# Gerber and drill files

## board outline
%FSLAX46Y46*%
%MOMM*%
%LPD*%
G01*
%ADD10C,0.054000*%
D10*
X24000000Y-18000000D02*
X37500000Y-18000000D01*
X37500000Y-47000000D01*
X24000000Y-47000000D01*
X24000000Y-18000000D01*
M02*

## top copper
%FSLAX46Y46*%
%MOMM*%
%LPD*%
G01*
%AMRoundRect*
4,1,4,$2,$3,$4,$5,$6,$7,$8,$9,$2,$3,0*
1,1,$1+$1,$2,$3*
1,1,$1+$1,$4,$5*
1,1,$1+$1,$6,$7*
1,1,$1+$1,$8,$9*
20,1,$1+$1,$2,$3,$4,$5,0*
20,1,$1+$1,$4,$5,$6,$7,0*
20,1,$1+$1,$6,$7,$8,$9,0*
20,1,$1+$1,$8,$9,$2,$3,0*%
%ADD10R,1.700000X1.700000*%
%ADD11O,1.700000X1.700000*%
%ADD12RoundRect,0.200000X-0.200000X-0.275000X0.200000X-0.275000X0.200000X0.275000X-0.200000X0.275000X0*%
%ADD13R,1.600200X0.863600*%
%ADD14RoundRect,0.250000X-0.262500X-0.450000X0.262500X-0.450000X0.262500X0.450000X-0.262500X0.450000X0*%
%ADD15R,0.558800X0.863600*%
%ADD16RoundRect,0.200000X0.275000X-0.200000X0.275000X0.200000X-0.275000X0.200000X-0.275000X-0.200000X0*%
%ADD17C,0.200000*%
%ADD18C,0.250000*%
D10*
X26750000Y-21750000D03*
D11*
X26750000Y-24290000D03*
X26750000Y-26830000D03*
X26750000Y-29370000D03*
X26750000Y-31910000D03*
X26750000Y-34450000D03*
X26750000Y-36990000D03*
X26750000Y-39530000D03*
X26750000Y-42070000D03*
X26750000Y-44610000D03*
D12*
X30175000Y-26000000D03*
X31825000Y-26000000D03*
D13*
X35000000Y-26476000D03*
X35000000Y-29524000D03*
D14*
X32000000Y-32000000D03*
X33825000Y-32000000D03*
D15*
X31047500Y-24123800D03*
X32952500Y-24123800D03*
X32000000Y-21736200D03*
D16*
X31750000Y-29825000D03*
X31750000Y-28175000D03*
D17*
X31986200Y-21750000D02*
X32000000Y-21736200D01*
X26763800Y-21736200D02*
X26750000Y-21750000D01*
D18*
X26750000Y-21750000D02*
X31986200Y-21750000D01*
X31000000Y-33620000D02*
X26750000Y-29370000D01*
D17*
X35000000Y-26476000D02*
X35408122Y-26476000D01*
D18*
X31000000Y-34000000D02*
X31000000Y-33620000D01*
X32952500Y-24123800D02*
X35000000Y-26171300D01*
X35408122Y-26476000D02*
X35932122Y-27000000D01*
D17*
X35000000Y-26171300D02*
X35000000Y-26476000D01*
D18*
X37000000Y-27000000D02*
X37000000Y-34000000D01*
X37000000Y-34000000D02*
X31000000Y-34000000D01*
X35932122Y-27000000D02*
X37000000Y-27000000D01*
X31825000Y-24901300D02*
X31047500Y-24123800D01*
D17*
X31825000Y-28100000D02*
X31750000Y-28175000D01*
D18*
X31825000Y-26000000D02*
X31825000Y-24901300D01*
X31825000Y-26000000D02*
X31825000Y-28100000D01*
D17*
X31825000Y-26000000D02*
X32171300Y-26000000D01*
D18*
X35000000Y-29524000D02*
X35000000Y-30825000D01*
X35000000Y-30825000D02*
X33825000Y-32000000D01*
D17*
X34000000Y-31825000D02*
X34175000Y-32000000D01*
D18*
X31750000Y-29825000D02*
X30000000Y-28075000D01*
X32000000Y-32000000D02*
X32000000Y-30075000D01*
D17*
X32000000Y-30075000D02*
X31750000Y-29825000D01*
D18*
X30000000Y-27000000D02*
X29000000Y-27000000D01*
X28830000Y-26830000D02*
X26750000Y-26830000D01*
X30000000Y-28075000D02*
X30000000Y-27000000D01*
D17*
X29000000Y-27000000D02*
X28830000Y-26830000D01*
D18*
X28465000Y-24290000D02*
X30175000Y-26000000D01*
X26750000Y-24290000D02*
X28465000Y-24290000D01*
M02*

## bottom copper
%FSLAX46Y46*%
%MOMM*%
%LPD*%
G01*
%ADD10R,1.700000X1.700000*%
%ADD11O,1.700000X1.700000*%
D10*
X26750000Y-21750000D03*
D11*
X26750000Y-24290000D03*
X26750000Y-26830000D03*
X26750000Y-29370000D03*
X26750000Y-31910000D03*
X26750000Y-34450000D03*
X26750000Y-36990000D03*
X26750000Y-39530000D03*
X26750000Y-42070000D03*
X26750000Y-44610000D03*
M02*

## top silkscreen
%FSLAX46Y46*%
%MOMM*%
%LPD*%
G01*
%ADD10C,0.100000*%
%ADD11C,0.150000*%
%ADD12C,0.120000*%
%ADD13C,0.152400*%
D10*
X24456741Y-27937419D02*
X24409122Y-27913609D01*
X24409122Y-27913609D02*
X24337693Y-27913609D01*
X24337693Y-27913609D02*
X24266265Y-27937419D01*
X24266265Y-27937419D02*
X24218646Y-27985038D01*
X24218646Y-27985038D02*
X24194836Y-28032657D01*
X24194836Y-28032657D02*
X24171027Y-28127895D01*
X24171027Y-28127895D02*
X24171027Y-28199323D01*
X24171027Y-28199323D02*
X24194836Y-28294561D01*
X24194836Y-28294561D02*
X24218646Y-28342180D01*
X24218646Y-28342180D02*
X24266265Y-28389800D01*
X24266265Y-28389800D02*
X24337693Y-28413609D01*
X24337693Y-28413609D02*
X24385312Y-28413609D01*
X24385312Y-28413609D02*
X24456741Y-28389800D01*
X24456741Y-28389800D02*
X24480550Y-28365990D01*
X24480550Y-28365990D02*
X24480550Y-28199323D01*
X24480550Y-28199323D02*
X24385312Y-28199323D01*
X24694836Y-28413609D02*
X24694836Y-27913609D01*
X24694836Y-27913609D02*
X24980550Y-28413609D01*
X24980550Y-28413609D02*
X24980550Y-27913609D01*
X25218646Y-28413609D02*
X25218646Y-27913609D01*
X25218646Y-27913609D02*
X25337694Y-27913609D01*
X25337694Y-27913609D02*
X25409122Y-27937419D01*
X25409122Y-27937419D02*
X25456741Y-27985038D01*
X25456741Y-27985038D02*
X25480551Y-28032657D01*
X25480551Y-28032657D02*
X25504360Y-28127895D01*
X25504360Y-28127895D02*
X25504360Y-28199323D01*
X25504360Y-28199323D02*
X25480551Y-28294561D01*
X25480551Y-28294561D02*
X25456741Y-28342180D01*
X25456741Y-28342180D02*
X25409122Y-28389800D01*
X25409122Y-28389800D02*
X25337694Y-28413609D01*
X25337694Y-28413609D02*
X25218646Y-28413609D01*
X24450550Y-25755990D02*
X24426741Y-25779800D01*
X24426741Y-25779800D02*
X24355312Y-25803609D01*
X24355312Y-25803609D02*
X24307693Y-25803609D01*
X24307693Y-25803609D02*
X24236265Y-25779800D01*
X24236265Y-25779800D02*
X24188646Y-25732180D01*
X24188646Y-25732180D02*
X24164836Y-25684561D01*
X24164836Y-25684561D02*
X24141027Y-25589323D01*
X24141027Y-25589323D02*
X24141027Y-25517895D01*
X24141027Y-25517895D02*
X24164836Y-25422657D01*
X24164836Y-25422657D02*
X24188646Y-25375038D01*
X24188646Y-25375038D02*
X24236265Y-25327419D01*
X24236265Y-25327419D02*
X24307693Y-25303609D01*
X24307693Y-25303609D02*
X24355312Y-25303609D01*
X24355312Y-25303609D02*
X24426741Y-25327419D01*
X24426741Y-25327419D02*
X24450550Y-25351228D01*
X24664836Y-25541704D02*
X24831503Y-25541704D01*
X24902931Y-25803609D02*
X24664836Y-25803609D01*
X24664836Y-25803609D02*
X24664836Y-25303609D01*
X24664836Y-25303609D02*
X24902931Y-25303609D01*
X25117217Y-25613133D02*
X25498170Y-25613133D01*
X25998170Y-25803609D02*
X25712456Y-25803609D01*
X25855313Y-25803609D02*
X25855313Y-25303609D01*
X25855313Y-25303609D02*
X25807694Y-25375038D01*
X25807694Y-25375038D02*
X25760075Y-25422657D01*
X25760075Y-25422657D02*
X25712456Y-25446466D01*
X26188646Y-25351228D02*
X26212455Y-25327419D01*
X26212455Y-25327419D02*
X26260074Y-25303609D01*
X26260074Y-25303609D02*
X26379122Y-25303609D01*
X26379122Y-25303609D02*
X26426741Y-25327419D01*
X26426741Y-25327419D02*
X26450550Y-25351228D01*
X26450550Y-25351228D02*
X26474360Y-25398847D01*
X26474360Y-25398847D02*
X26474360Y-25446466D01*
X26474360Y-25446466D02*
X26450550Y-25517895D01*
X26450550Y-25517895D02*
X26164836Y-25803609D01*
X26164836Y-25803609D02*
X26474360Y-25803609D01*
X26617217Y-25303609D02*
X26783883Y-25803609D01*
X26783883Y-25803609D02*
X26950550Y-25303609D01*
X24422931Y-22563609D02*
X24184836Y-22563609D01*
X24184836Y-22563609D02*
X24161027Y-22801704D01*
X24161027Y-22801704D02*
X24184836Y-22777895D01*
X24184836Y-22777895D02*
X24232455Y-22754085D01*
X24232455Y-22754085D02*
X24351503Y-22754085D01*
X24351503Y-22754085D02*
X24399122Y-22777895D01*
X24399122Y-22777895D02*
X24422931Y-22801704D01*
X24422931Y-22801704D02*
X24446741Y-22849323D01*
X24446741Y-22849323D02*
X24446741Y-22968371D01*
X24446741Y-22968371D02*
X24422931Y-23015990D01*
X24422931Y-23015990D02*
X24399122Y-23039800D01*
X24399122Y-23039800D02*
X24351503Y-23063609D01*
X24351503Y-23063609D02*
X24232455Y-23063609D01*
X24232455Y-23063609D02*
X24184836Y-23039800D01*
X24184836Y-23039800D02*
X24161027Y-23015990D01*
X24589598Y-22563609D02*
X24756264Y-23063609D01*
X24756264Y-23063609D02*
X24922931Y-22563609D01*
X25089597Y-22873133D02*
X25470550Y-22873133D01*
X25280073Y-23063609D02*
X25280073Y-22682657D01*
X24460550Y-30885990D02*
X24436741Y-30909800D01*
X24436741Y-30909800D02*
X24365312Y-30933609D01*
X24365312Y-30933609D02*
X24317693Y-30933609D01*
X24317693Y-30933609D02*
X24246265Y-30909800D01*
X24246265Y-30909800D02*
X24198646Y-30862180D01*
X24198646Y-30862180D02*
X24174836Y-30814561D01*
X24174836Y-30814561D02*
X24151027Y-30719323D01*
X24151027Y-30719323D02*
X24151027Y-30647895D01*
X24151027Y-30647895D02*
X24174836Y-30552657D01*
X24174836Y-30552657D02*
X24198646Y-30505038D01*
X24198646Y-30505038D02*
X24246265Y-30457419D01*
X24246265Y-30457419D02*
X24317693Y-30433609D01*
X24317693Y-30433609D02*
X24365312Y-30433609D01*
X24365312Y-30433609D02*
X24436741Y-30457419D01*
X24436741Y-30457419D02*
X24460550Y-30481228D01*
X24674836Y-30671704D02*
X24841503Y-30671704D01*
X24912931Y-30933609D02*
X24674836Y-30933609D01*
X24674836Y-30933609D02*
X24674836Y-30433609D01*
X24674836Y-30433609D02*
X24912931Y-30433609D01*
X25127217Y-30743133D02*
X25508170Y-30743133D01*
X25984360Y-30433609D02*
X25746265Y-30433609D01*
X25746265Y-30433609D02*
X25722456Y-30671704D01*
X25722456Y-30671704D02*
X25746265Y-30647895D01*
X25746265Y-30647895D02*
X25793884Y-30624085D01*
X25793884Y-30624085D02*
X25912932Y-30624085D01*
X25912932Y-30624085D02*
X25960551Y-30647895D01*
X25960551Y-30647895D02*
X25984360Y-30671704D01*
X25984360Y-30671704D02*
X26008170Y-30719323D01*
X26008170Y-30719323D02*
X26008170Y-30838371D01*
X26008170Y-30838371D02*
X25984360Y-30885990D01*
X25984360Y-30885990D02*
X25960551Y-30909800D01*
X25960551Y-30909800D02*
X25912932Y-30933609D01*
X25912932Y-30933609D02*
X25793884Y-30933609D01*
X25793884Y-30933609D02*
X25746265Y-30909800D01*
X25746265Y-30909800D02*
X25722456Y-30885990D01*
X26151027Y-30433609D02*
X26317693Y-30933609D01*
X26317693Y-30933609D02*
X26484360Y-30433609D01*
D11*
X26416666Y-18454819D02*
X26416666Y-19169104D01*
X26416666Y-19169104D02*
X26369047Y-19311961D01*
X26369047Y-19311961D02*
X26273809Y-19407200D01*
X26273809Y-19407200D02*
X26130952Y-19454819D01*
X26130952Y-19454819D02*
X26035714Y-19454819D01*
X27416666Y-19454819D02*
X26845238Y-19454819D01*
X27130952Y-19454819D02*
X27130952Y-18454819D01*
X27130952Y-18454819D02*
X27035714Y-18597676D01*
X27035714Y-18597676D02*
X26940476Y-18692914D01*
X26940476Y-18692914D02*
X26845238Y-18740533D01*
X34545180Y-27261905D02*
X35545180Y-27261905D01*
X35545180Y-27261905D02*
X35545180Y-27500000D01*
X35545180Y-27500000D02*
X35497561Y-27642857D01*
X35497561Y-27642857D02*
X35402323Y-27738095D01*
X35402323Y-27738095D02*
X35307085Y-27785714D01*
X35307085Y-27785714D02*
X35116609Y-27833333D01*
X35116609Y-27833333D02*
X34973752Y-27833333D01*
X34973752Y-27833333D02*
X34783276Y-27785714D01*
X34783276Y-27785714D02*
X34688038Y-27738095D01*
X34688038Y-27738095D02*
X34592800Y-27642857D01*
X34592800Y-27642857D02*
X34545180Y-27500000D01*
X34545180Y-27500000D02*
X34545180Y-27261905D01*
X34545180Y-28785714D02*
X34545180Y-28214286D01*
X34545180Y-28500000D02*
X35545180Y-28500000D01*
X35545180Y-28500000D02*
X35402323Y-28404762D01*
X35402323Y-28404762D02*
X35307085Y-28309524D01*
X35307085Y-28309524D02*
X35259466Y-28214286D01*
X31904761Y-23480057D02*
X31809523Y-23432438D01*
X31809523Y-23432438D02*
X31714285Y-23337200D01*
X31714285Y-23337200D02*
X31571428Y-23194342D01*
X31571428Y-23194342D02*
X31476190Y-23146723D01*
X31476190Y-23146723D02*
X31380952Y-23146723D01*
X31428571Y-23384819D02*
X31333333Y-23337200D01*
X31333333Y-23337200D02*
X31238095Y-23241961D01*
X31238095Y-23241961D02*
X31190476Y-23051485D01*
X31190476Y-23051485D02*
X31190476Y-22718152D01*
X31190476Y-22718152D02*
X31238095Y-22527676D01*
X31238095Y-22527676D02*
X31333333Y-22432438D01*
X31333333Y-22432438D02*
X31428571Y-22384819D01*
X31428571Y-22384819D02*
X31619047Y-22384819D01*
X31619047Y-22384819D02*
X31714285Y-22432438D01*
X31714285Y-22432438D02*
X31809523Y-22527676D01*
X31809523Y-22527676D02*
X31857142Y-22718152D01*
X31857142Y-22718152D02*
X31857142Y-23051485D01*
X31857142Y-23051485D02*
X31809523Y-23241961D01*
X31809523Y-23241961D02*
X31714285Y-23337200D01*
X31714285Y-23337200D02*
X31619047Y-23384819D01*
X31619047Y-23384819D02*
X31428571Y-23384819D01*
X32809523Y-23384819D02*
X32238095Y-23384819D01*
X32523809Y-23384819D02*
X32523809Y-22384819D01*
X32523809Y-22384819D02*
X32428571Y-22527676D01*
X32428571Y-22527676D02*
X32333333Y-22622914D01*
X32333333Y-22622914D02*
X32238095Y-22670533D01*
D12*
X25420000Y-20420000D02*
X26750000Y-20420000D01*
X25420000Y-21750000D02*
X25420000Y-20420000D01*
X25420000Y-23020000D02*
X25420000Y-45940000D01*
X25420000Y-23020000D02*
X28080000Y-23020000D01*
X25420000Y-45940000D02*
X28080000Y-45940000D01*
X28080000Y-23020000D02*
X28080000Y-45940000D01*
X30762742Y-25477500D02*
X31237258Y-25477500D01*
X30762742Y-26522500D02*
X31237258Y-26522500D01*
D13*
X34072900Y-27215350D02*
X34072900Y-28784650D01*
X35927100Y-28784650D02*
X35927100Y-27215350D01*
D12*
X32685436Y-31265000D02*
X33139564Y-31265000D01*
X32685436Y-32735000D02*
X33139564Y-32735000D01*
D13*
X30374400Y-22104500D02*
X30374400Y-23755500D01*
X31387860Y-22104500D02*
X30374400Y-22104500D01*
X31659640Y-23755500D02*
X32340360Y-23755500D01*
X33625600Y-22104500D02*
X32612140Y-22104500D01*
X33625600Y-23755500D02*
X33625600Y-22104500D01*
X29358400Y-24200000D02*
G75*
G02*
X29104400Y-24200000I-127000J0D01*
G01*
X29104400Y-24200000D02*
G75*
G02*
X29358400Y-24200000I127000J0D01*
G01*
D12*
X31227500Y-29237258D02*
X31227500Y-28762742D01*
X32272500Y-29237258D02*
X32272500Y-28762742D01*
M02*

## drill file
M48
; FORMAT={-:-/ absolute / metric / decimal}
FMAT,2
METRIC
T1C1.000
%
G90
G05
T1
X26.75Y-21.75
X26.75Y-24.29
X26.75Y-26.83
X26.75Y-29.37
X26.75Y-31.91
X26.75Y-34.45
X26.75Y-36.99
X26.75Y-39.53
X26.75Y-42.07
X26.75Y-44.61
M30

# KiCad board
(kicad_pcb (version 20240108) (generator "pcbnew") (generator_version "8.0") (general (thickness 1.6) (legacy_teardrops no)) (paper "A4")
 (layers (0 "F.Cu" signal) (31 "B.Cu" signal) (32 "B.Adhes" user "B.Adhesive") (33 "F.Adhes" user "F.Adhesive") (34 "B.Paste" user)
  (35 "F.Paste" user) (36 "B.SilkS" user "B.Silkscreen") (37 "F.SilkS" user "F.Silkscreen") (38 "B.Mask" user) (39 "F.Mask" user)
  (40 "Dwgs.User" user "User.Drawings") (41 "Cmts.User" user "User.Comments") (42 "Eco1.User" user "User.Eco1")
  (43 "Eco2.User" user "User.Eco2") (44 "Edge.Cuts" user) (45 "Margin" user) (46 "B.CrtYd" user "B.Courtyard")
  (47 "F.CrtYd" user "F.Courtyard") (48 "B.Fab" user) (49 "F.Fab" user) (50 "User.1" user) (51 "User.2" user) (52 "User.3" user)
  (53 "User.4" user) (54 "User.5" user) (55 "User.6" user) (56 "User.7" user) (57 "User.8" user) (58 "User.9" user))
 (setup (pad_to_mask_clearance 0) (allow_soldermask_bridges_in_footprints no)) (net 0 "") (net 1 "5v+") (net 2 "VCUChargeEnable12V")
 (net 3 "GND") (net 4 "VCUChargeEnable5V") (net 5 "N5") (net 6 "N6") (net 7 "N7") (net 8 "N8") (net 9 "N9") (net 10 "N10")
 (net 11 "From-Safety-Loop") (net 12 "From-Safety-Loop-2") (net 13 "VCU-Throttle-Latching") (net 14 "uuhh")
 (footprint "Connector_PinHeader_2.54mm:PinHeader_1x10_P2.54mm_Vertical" (layer "F.Cu") (at 26.75 21.75)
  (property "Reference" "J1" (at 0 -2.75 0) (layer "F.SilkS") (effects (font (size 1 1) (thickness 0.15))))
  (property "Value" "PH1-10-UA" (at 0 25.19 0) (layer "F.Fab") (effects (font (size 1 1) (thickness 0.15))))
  (fp_line (start -1.33 -1.33) (end 0 -1.33) (stroke (width 0.12) (type solid)) (layer "F.SilkS"))
  (fp_line (start -1.33 0) (end -1.33 -1.33) (stroke (width 0.12) (type solid)) (layer "F.SilkS"))
  (fp_line (start -1.33 1.27) (end -1.33 24.19) (stroke (width 0.12) (type solid)) (layer "F.SilkS"))
  (fp_line (start -1.33 1.27) (end 1.33 1.27) (stroke (width 0.12) (type solid)) (layer "F.SilkS"))
  (fp_line (start -1.33 24.19) (end 1.33 24.19) (stroke (width 0.12) (type solid)) (layer "F.SilkS"))
  (fp_line (start 1.33 1.27) (end 1.33 24.19) (stroke (width 0.12) (type solid)) (layer "F.SilkS"))
  (pad "1" thru_hole rect (at 0 0) (size 1.7 1.7) (drill 1) (layers "*.Cu" "*.Mask") (remove_unused_layers no) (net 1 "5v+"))
  (pad "2" thru_hole oval (at 0 2.54) (size 1.7 1.7) (drill 1) (layers "*.Cu" "*.Mask") (remove_unused_layers no)
   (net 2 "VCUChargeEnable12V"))
  (pad "3" thru_hole oval (at 0 5.08) (size 1.7 1.7) (drill 1) (layers "*.Cu" "*.Mask") (remove_unused_layers no) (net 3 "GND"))
  (pad "4" thru_hole oval (at 0 7.62) (size 1.7 1.7) (drill 1) (layers "*.Cu" "*.Mask") (remove_unused_layers no)
   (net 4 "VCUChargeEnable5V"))
  (pad "5" thru_hole oval (at 0 10.16) (size 1.7 1.7) (drill 1) (layers "*.Cu" "*.Mask") (remove_unused_layers no) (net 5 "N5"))
  (pad "6" thru_hole oval (at 0 12.7) (size 1.7 1.7) (drill 1) (layers "*.Cu" "*.Mask") (remove_unused_layers no) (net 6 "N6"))
  (pad "7" thru_hole oval (at 0 15.24) (size 1.7 1.7) (drill 1) (layers "*.Cu" "*.Mask") (remove_unused_layers no) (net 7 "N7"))
  (pad "8" thru_hole oval (at 0 17.78) (size 1.7 1.7) (drill 1) (layers "*.Cu" "*.Mask") (remove_unused_layers no) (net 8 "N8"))
  (pad "9" thru_hole oval (at 0 20.32) (size 1.7 1.7) (drill 1) (layers "*.Cu" "*.Mask") (remove_unused_layers no) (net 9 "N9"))
  (pad "10" thru_hole oval (at 0 22.86) (size 1.7 1.7) (drill 1) (layers "*.Cu" "*.Mask") (remove_unused_layers no) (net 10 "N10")))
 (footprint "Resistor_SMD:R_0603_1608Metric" (layer "F.Cu") (at 31 26)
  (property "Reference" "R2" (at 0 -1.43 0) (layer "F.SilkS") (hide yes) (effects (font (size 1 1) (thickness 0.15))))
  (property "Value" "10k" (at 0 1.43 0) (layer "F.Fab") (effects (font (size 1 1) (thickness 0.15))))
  (fp_line (start -0.237258 -0.5225) (end 0.237258 -0.5225) (stroke (width 0.12) (type solid)) (layer "F.SilkS"))
  (fp_line (start -0.237258 0.5225) (end 0.237258 0.5225) (stroke (width 0.12) (type solid)) (layer "F.SilkS"))
  (pad "1" smd roundrect (at -0.825 0) (size 0.8 0.95) (layers "F.Cu" "F.Paste" "F.Mask") (roundrect_rratio 0.25)
   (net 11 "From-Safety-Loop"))
  (pad "2" smd roundrect (at 0.825 0) (size 0.8 0.95) (layers "F.Cu" "F.Paste" "F.Mask") (roundrect_rratio 0.25)
   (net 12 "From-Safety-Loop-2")))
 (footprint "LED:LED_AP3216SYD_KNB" (layer "F.Cu") (at 35 28 -90)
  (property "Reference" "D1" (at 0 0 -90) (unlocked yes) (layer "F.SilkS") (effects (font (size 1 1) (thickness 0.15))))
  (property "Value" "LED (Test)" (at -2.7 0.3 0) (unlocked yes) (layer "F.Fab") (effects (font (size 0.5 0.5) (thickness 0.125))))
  (fp_line (start -0.78465 0.9271) (end 0.78465 0.9271) (stroke (width 0.1524) (type solid)) (layer "F.SilkS"))
  (fp_line (start 0.78465 -0.9271) (end -0.78465 -0.9271) (stroke (width 0.1524) (type solid)) (layer "F.SilkS"))
  (pad "1" smd rect (at -1.524 0 270) (size 0.8636 1.6002) (layers "F.Cu" "F.Paste" "F.Mask") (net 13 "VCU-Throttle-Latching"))
  (pad "2" smd rect (at 1.524 0 270) (size 0.8636 1.6002) (layers "F.Cu" "F.Paste" "F.Mask") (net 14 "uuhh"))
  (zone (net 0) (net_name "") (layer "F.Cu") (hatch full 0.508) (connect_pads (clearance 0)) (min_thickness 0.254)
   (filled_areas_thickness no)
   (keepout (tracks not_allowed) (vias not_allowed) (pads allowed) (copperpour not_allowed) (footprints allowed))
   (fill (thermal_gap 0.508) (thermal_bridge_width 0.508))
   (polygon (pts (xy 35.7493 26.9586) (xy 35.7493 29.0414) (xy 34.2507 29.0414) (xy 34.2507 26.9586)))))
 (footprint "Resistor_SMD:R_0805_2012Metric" (layer "F.Cu") (at 32.9125 32)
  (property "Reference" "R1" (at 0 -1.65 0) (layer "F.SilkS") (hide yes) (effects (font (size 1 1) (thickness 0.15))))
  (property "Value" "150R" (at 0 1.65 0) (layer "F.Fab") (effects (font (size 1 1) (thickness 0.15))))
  (fp_line (start -0.227064 -0.735) (end 0.227064 -0.735) (stroke (width 0.12) (type solid)) (layer "F.SilkS"))
  (fp_line (start -0.227064 0.735) (end 0.227064 0.735) (stroke (width 0.12) (type solid)) (layer "F.SilkS"))
  (pad "1" smd roundrect (at -0.9125 0) (size 1.025 1.4) (layers "F.Cu" "F.Paste" "F.Mask") (roundrect_rratio 0.243902) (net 3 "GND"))
  (pad "2" smd roundrect (at 0.9125 0) (size 1.025 1.4) (layers "F.Cu" "F.Paste" "F.Mask") (roundrect_rratio 0.243902) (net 14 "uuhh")))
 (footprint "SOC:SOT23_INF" (layer "F.Cu") (at 32 22.93)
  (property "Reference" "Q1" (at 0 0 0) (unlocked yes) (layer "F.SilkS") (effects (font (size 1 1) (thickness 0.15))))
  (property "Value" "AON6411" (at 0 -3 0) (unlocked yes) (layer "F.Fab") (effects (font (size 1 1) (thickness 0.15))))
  (fp_line (start -1.6256 -0.8255) (end -1.6256 0.8255) (stroke (width 0.1524) (type solid)) (layer "F.SilkS"))
  (fp_line (start -0.61214 -0.8255) (end -1.6256 -0.8255) (stroke (width 0.1524) (type solid)) (layer "F.SilkS"))
  (fp_line (start -0.34036 0.8255) (end 0.34036 0.8255) (stroke (width 0.1524) (type solid)) (layer "F.SilkS"))
  (fp_line (start 1.6256 -0.8255) (end 0.61214 -0.8255) (stroke (width 0.1524) (type solid)) (layer "F.SilkS"))
  (fp_line (start 1.6256 0.8255) (end 1.6256 -0.8255) (stroke (width 0.1524) (type solid)) (layer "F.SilkS"))
  (fp_circle (center -2.7686 1.27) (end -2.6416 1.27) (stroke (width 0.1524) (type solid)) (fill none) (layer "F.SilkS"))
  (pad "1" smd rect (at -0.9525 1.1938) (size 0.5588 0.8636) (layers "F.Cu" "F.Paste" "F.Mask") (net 12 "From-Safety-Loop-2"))
  (pad "2" smd rect (at 0.9525 1.1938) (size 0.5588 0.8636) (layers "F.Cu" "F.Paste" "F.Mask") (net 13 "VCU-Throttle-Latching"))
  (pad "3" smd rect (at 0 -1.1938) (size 0.5588 0.8636) (layers "F.Cu" "F.Paste" "F.Mask") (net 1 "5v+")))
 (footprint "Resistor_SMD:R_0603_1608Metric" (layer "F.Cu") (at 31.75 29 90)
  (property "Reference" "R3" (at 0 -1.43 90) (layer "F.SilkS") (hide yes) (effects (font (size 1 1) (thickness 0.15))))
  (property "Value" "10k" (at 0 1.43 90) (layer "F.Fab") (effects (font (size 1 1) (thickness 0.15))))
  (fp_line (start -0.237258 -0.5225) (end 0.237258 -0.5225) (stroke (width 0.12) (type solid)) (layer "F.SilkS"))
  (fp_line (start -0.237258 0.5225) (end 0.237258 0.5225) (stroke (width 0.12) (type solid)) (layer "F.SilkS"))
  (pad "1" smd roundrect (at -0.825 0 90) (size 0.8 0.95) (layers "F.Cu" "F.Paste" "F.Mask") (roundrect_rratio 0.25) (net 3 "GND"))
  (pad "2" smd roundrect (at 0.825 0 90) (size 0.8 0.95) (layers "F.Cu" "F.Paste" "F.Mask") (roundrect_rratio 0.25)
   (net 12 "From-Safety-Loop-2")))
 (gr_rect (start 24 18) (end 37.5 47) (stroke (width 0.054) (type default)) (fill none) (layer "Edge.Cuts"))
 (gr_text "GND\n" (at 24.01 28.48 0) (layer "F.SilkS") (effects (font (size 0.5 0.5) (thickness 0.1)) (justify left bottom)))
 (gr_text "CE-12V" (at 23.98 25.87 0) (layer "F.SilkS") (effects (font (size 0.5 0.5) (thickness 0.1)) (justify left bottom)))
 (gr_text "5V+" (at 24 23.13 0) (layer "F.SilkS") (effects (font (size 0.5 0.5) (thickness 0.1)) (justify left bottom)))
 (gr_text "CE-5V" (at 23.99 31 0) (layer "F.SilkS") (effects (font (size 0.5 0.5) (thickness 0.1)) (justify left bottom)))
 (segment (start 31.9862 21.75) (end 32 21.7362) (width 0.2) (layer "F.Cu") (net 1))
 (segment (start 26.7638 21.7362) (end 26.75 21.75) (width 0.2) (layer "F.Cu") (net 1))
 (segment (start 26.75 21.75) (end 31.9862 21.75) (width 0.25) (layer "F.Cu") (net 1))
 (segment (start 31 33.62) (end 26.75 29.37) (width 0.25) (layer "F.Cu") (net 13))
 (segment (start 35 26.476) (end 35.408122 26.476) (width 0.2) (layer "F.Cu") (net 13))
 (segment (start 31 34) (end 31 33.62) (width 0.25) (layer "F.Cu") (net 13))
 (segment (start 32.9525 24.1238) (end 35 26.1713) (width 0.25) (layer "F.Cu") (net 13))
 (segment (start 35.408122 26.476) (end 35.932122 27) (width 0.25) (layer "F.Cu") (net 13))
 (segment (start 35 26.1713) (end 35 26.476) (width 0.2) (layer "F.Cu") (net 13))
 (segment (start 37 27) (end 37 34) (width 0.25) (layer "F.Cu") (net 13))
 (segment (start 37 34) (end 31 34) (width 0.25) (layer "F.Cu") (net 13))
 (segment (start 35.932122 27) (end 37 27) (width 0.25) (layer "F.Cu") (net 13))
 (segment (start 31.825 24.9013) (end 31.0475 24.1238) (width 0.25) (layer "F.Cu") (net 12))
 (segment (start 31.825 28.1) (end 31.75 28.175) (width 0.2) (layer "F.Cu") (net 12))
 (segment (start 31.825 26) (end 31.825 24.9013) (width 0.25) (layer "F.Cu") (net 12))
 (segment (start 31.825 26) (end 31.825 28.1) (width 0.25) (layer "F.Cu") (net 12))
 (segment (start 31.825 26) (end 32.1713 26) (width 0.2) (layer "F.Cu") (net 12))
 (segment (start 35 29.524) (end 35 30.825) (width 0.25) (layer "F.Cu") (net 14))
 (segment (start 35 30.825) (end 33.825 32) (width 0.25) (layer "F.Cu") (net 14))
 (segment (start 34 31.825) (end 34.175 32) (width 0.2) (layer "F.Cu") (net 14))
 (segment (start 31.75 29.825) (end 30 28.075) (width 0.25) (layer "F.Cu") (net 3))
 (segment (start 32 32) (end 32 30.075) (width 0.25) (layer "F.Cu") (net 3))
 (segment (start 32 30.075) (end 31.75 29.825) (width 0.2) (layer "F.Cu") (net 3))
 (segment (start 30 27) (end 29 27) (width 0.25) (layer "F.Cu") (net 3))
 (segment (start 28.83 26.83) (end 26.75 26.83) (width 0.25) (layer "F.Cu") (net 3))
 (segment (start 30 28.075) (end 30 27) (width 0.25) (layer "F.Cu") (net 3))
 (segment (start 29 27) (end 28.83 26.83) (width 0.2) (layer "F.Cu") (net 3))
 (segment (start 28.465 24.29) (end 30.175 26) (width 0.25) (layer "F.Cu") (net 11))
 (segment (start 26.75 24.29) (end 28.465 24.29) (width 0.25) (layer "F.Cu") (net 11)))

